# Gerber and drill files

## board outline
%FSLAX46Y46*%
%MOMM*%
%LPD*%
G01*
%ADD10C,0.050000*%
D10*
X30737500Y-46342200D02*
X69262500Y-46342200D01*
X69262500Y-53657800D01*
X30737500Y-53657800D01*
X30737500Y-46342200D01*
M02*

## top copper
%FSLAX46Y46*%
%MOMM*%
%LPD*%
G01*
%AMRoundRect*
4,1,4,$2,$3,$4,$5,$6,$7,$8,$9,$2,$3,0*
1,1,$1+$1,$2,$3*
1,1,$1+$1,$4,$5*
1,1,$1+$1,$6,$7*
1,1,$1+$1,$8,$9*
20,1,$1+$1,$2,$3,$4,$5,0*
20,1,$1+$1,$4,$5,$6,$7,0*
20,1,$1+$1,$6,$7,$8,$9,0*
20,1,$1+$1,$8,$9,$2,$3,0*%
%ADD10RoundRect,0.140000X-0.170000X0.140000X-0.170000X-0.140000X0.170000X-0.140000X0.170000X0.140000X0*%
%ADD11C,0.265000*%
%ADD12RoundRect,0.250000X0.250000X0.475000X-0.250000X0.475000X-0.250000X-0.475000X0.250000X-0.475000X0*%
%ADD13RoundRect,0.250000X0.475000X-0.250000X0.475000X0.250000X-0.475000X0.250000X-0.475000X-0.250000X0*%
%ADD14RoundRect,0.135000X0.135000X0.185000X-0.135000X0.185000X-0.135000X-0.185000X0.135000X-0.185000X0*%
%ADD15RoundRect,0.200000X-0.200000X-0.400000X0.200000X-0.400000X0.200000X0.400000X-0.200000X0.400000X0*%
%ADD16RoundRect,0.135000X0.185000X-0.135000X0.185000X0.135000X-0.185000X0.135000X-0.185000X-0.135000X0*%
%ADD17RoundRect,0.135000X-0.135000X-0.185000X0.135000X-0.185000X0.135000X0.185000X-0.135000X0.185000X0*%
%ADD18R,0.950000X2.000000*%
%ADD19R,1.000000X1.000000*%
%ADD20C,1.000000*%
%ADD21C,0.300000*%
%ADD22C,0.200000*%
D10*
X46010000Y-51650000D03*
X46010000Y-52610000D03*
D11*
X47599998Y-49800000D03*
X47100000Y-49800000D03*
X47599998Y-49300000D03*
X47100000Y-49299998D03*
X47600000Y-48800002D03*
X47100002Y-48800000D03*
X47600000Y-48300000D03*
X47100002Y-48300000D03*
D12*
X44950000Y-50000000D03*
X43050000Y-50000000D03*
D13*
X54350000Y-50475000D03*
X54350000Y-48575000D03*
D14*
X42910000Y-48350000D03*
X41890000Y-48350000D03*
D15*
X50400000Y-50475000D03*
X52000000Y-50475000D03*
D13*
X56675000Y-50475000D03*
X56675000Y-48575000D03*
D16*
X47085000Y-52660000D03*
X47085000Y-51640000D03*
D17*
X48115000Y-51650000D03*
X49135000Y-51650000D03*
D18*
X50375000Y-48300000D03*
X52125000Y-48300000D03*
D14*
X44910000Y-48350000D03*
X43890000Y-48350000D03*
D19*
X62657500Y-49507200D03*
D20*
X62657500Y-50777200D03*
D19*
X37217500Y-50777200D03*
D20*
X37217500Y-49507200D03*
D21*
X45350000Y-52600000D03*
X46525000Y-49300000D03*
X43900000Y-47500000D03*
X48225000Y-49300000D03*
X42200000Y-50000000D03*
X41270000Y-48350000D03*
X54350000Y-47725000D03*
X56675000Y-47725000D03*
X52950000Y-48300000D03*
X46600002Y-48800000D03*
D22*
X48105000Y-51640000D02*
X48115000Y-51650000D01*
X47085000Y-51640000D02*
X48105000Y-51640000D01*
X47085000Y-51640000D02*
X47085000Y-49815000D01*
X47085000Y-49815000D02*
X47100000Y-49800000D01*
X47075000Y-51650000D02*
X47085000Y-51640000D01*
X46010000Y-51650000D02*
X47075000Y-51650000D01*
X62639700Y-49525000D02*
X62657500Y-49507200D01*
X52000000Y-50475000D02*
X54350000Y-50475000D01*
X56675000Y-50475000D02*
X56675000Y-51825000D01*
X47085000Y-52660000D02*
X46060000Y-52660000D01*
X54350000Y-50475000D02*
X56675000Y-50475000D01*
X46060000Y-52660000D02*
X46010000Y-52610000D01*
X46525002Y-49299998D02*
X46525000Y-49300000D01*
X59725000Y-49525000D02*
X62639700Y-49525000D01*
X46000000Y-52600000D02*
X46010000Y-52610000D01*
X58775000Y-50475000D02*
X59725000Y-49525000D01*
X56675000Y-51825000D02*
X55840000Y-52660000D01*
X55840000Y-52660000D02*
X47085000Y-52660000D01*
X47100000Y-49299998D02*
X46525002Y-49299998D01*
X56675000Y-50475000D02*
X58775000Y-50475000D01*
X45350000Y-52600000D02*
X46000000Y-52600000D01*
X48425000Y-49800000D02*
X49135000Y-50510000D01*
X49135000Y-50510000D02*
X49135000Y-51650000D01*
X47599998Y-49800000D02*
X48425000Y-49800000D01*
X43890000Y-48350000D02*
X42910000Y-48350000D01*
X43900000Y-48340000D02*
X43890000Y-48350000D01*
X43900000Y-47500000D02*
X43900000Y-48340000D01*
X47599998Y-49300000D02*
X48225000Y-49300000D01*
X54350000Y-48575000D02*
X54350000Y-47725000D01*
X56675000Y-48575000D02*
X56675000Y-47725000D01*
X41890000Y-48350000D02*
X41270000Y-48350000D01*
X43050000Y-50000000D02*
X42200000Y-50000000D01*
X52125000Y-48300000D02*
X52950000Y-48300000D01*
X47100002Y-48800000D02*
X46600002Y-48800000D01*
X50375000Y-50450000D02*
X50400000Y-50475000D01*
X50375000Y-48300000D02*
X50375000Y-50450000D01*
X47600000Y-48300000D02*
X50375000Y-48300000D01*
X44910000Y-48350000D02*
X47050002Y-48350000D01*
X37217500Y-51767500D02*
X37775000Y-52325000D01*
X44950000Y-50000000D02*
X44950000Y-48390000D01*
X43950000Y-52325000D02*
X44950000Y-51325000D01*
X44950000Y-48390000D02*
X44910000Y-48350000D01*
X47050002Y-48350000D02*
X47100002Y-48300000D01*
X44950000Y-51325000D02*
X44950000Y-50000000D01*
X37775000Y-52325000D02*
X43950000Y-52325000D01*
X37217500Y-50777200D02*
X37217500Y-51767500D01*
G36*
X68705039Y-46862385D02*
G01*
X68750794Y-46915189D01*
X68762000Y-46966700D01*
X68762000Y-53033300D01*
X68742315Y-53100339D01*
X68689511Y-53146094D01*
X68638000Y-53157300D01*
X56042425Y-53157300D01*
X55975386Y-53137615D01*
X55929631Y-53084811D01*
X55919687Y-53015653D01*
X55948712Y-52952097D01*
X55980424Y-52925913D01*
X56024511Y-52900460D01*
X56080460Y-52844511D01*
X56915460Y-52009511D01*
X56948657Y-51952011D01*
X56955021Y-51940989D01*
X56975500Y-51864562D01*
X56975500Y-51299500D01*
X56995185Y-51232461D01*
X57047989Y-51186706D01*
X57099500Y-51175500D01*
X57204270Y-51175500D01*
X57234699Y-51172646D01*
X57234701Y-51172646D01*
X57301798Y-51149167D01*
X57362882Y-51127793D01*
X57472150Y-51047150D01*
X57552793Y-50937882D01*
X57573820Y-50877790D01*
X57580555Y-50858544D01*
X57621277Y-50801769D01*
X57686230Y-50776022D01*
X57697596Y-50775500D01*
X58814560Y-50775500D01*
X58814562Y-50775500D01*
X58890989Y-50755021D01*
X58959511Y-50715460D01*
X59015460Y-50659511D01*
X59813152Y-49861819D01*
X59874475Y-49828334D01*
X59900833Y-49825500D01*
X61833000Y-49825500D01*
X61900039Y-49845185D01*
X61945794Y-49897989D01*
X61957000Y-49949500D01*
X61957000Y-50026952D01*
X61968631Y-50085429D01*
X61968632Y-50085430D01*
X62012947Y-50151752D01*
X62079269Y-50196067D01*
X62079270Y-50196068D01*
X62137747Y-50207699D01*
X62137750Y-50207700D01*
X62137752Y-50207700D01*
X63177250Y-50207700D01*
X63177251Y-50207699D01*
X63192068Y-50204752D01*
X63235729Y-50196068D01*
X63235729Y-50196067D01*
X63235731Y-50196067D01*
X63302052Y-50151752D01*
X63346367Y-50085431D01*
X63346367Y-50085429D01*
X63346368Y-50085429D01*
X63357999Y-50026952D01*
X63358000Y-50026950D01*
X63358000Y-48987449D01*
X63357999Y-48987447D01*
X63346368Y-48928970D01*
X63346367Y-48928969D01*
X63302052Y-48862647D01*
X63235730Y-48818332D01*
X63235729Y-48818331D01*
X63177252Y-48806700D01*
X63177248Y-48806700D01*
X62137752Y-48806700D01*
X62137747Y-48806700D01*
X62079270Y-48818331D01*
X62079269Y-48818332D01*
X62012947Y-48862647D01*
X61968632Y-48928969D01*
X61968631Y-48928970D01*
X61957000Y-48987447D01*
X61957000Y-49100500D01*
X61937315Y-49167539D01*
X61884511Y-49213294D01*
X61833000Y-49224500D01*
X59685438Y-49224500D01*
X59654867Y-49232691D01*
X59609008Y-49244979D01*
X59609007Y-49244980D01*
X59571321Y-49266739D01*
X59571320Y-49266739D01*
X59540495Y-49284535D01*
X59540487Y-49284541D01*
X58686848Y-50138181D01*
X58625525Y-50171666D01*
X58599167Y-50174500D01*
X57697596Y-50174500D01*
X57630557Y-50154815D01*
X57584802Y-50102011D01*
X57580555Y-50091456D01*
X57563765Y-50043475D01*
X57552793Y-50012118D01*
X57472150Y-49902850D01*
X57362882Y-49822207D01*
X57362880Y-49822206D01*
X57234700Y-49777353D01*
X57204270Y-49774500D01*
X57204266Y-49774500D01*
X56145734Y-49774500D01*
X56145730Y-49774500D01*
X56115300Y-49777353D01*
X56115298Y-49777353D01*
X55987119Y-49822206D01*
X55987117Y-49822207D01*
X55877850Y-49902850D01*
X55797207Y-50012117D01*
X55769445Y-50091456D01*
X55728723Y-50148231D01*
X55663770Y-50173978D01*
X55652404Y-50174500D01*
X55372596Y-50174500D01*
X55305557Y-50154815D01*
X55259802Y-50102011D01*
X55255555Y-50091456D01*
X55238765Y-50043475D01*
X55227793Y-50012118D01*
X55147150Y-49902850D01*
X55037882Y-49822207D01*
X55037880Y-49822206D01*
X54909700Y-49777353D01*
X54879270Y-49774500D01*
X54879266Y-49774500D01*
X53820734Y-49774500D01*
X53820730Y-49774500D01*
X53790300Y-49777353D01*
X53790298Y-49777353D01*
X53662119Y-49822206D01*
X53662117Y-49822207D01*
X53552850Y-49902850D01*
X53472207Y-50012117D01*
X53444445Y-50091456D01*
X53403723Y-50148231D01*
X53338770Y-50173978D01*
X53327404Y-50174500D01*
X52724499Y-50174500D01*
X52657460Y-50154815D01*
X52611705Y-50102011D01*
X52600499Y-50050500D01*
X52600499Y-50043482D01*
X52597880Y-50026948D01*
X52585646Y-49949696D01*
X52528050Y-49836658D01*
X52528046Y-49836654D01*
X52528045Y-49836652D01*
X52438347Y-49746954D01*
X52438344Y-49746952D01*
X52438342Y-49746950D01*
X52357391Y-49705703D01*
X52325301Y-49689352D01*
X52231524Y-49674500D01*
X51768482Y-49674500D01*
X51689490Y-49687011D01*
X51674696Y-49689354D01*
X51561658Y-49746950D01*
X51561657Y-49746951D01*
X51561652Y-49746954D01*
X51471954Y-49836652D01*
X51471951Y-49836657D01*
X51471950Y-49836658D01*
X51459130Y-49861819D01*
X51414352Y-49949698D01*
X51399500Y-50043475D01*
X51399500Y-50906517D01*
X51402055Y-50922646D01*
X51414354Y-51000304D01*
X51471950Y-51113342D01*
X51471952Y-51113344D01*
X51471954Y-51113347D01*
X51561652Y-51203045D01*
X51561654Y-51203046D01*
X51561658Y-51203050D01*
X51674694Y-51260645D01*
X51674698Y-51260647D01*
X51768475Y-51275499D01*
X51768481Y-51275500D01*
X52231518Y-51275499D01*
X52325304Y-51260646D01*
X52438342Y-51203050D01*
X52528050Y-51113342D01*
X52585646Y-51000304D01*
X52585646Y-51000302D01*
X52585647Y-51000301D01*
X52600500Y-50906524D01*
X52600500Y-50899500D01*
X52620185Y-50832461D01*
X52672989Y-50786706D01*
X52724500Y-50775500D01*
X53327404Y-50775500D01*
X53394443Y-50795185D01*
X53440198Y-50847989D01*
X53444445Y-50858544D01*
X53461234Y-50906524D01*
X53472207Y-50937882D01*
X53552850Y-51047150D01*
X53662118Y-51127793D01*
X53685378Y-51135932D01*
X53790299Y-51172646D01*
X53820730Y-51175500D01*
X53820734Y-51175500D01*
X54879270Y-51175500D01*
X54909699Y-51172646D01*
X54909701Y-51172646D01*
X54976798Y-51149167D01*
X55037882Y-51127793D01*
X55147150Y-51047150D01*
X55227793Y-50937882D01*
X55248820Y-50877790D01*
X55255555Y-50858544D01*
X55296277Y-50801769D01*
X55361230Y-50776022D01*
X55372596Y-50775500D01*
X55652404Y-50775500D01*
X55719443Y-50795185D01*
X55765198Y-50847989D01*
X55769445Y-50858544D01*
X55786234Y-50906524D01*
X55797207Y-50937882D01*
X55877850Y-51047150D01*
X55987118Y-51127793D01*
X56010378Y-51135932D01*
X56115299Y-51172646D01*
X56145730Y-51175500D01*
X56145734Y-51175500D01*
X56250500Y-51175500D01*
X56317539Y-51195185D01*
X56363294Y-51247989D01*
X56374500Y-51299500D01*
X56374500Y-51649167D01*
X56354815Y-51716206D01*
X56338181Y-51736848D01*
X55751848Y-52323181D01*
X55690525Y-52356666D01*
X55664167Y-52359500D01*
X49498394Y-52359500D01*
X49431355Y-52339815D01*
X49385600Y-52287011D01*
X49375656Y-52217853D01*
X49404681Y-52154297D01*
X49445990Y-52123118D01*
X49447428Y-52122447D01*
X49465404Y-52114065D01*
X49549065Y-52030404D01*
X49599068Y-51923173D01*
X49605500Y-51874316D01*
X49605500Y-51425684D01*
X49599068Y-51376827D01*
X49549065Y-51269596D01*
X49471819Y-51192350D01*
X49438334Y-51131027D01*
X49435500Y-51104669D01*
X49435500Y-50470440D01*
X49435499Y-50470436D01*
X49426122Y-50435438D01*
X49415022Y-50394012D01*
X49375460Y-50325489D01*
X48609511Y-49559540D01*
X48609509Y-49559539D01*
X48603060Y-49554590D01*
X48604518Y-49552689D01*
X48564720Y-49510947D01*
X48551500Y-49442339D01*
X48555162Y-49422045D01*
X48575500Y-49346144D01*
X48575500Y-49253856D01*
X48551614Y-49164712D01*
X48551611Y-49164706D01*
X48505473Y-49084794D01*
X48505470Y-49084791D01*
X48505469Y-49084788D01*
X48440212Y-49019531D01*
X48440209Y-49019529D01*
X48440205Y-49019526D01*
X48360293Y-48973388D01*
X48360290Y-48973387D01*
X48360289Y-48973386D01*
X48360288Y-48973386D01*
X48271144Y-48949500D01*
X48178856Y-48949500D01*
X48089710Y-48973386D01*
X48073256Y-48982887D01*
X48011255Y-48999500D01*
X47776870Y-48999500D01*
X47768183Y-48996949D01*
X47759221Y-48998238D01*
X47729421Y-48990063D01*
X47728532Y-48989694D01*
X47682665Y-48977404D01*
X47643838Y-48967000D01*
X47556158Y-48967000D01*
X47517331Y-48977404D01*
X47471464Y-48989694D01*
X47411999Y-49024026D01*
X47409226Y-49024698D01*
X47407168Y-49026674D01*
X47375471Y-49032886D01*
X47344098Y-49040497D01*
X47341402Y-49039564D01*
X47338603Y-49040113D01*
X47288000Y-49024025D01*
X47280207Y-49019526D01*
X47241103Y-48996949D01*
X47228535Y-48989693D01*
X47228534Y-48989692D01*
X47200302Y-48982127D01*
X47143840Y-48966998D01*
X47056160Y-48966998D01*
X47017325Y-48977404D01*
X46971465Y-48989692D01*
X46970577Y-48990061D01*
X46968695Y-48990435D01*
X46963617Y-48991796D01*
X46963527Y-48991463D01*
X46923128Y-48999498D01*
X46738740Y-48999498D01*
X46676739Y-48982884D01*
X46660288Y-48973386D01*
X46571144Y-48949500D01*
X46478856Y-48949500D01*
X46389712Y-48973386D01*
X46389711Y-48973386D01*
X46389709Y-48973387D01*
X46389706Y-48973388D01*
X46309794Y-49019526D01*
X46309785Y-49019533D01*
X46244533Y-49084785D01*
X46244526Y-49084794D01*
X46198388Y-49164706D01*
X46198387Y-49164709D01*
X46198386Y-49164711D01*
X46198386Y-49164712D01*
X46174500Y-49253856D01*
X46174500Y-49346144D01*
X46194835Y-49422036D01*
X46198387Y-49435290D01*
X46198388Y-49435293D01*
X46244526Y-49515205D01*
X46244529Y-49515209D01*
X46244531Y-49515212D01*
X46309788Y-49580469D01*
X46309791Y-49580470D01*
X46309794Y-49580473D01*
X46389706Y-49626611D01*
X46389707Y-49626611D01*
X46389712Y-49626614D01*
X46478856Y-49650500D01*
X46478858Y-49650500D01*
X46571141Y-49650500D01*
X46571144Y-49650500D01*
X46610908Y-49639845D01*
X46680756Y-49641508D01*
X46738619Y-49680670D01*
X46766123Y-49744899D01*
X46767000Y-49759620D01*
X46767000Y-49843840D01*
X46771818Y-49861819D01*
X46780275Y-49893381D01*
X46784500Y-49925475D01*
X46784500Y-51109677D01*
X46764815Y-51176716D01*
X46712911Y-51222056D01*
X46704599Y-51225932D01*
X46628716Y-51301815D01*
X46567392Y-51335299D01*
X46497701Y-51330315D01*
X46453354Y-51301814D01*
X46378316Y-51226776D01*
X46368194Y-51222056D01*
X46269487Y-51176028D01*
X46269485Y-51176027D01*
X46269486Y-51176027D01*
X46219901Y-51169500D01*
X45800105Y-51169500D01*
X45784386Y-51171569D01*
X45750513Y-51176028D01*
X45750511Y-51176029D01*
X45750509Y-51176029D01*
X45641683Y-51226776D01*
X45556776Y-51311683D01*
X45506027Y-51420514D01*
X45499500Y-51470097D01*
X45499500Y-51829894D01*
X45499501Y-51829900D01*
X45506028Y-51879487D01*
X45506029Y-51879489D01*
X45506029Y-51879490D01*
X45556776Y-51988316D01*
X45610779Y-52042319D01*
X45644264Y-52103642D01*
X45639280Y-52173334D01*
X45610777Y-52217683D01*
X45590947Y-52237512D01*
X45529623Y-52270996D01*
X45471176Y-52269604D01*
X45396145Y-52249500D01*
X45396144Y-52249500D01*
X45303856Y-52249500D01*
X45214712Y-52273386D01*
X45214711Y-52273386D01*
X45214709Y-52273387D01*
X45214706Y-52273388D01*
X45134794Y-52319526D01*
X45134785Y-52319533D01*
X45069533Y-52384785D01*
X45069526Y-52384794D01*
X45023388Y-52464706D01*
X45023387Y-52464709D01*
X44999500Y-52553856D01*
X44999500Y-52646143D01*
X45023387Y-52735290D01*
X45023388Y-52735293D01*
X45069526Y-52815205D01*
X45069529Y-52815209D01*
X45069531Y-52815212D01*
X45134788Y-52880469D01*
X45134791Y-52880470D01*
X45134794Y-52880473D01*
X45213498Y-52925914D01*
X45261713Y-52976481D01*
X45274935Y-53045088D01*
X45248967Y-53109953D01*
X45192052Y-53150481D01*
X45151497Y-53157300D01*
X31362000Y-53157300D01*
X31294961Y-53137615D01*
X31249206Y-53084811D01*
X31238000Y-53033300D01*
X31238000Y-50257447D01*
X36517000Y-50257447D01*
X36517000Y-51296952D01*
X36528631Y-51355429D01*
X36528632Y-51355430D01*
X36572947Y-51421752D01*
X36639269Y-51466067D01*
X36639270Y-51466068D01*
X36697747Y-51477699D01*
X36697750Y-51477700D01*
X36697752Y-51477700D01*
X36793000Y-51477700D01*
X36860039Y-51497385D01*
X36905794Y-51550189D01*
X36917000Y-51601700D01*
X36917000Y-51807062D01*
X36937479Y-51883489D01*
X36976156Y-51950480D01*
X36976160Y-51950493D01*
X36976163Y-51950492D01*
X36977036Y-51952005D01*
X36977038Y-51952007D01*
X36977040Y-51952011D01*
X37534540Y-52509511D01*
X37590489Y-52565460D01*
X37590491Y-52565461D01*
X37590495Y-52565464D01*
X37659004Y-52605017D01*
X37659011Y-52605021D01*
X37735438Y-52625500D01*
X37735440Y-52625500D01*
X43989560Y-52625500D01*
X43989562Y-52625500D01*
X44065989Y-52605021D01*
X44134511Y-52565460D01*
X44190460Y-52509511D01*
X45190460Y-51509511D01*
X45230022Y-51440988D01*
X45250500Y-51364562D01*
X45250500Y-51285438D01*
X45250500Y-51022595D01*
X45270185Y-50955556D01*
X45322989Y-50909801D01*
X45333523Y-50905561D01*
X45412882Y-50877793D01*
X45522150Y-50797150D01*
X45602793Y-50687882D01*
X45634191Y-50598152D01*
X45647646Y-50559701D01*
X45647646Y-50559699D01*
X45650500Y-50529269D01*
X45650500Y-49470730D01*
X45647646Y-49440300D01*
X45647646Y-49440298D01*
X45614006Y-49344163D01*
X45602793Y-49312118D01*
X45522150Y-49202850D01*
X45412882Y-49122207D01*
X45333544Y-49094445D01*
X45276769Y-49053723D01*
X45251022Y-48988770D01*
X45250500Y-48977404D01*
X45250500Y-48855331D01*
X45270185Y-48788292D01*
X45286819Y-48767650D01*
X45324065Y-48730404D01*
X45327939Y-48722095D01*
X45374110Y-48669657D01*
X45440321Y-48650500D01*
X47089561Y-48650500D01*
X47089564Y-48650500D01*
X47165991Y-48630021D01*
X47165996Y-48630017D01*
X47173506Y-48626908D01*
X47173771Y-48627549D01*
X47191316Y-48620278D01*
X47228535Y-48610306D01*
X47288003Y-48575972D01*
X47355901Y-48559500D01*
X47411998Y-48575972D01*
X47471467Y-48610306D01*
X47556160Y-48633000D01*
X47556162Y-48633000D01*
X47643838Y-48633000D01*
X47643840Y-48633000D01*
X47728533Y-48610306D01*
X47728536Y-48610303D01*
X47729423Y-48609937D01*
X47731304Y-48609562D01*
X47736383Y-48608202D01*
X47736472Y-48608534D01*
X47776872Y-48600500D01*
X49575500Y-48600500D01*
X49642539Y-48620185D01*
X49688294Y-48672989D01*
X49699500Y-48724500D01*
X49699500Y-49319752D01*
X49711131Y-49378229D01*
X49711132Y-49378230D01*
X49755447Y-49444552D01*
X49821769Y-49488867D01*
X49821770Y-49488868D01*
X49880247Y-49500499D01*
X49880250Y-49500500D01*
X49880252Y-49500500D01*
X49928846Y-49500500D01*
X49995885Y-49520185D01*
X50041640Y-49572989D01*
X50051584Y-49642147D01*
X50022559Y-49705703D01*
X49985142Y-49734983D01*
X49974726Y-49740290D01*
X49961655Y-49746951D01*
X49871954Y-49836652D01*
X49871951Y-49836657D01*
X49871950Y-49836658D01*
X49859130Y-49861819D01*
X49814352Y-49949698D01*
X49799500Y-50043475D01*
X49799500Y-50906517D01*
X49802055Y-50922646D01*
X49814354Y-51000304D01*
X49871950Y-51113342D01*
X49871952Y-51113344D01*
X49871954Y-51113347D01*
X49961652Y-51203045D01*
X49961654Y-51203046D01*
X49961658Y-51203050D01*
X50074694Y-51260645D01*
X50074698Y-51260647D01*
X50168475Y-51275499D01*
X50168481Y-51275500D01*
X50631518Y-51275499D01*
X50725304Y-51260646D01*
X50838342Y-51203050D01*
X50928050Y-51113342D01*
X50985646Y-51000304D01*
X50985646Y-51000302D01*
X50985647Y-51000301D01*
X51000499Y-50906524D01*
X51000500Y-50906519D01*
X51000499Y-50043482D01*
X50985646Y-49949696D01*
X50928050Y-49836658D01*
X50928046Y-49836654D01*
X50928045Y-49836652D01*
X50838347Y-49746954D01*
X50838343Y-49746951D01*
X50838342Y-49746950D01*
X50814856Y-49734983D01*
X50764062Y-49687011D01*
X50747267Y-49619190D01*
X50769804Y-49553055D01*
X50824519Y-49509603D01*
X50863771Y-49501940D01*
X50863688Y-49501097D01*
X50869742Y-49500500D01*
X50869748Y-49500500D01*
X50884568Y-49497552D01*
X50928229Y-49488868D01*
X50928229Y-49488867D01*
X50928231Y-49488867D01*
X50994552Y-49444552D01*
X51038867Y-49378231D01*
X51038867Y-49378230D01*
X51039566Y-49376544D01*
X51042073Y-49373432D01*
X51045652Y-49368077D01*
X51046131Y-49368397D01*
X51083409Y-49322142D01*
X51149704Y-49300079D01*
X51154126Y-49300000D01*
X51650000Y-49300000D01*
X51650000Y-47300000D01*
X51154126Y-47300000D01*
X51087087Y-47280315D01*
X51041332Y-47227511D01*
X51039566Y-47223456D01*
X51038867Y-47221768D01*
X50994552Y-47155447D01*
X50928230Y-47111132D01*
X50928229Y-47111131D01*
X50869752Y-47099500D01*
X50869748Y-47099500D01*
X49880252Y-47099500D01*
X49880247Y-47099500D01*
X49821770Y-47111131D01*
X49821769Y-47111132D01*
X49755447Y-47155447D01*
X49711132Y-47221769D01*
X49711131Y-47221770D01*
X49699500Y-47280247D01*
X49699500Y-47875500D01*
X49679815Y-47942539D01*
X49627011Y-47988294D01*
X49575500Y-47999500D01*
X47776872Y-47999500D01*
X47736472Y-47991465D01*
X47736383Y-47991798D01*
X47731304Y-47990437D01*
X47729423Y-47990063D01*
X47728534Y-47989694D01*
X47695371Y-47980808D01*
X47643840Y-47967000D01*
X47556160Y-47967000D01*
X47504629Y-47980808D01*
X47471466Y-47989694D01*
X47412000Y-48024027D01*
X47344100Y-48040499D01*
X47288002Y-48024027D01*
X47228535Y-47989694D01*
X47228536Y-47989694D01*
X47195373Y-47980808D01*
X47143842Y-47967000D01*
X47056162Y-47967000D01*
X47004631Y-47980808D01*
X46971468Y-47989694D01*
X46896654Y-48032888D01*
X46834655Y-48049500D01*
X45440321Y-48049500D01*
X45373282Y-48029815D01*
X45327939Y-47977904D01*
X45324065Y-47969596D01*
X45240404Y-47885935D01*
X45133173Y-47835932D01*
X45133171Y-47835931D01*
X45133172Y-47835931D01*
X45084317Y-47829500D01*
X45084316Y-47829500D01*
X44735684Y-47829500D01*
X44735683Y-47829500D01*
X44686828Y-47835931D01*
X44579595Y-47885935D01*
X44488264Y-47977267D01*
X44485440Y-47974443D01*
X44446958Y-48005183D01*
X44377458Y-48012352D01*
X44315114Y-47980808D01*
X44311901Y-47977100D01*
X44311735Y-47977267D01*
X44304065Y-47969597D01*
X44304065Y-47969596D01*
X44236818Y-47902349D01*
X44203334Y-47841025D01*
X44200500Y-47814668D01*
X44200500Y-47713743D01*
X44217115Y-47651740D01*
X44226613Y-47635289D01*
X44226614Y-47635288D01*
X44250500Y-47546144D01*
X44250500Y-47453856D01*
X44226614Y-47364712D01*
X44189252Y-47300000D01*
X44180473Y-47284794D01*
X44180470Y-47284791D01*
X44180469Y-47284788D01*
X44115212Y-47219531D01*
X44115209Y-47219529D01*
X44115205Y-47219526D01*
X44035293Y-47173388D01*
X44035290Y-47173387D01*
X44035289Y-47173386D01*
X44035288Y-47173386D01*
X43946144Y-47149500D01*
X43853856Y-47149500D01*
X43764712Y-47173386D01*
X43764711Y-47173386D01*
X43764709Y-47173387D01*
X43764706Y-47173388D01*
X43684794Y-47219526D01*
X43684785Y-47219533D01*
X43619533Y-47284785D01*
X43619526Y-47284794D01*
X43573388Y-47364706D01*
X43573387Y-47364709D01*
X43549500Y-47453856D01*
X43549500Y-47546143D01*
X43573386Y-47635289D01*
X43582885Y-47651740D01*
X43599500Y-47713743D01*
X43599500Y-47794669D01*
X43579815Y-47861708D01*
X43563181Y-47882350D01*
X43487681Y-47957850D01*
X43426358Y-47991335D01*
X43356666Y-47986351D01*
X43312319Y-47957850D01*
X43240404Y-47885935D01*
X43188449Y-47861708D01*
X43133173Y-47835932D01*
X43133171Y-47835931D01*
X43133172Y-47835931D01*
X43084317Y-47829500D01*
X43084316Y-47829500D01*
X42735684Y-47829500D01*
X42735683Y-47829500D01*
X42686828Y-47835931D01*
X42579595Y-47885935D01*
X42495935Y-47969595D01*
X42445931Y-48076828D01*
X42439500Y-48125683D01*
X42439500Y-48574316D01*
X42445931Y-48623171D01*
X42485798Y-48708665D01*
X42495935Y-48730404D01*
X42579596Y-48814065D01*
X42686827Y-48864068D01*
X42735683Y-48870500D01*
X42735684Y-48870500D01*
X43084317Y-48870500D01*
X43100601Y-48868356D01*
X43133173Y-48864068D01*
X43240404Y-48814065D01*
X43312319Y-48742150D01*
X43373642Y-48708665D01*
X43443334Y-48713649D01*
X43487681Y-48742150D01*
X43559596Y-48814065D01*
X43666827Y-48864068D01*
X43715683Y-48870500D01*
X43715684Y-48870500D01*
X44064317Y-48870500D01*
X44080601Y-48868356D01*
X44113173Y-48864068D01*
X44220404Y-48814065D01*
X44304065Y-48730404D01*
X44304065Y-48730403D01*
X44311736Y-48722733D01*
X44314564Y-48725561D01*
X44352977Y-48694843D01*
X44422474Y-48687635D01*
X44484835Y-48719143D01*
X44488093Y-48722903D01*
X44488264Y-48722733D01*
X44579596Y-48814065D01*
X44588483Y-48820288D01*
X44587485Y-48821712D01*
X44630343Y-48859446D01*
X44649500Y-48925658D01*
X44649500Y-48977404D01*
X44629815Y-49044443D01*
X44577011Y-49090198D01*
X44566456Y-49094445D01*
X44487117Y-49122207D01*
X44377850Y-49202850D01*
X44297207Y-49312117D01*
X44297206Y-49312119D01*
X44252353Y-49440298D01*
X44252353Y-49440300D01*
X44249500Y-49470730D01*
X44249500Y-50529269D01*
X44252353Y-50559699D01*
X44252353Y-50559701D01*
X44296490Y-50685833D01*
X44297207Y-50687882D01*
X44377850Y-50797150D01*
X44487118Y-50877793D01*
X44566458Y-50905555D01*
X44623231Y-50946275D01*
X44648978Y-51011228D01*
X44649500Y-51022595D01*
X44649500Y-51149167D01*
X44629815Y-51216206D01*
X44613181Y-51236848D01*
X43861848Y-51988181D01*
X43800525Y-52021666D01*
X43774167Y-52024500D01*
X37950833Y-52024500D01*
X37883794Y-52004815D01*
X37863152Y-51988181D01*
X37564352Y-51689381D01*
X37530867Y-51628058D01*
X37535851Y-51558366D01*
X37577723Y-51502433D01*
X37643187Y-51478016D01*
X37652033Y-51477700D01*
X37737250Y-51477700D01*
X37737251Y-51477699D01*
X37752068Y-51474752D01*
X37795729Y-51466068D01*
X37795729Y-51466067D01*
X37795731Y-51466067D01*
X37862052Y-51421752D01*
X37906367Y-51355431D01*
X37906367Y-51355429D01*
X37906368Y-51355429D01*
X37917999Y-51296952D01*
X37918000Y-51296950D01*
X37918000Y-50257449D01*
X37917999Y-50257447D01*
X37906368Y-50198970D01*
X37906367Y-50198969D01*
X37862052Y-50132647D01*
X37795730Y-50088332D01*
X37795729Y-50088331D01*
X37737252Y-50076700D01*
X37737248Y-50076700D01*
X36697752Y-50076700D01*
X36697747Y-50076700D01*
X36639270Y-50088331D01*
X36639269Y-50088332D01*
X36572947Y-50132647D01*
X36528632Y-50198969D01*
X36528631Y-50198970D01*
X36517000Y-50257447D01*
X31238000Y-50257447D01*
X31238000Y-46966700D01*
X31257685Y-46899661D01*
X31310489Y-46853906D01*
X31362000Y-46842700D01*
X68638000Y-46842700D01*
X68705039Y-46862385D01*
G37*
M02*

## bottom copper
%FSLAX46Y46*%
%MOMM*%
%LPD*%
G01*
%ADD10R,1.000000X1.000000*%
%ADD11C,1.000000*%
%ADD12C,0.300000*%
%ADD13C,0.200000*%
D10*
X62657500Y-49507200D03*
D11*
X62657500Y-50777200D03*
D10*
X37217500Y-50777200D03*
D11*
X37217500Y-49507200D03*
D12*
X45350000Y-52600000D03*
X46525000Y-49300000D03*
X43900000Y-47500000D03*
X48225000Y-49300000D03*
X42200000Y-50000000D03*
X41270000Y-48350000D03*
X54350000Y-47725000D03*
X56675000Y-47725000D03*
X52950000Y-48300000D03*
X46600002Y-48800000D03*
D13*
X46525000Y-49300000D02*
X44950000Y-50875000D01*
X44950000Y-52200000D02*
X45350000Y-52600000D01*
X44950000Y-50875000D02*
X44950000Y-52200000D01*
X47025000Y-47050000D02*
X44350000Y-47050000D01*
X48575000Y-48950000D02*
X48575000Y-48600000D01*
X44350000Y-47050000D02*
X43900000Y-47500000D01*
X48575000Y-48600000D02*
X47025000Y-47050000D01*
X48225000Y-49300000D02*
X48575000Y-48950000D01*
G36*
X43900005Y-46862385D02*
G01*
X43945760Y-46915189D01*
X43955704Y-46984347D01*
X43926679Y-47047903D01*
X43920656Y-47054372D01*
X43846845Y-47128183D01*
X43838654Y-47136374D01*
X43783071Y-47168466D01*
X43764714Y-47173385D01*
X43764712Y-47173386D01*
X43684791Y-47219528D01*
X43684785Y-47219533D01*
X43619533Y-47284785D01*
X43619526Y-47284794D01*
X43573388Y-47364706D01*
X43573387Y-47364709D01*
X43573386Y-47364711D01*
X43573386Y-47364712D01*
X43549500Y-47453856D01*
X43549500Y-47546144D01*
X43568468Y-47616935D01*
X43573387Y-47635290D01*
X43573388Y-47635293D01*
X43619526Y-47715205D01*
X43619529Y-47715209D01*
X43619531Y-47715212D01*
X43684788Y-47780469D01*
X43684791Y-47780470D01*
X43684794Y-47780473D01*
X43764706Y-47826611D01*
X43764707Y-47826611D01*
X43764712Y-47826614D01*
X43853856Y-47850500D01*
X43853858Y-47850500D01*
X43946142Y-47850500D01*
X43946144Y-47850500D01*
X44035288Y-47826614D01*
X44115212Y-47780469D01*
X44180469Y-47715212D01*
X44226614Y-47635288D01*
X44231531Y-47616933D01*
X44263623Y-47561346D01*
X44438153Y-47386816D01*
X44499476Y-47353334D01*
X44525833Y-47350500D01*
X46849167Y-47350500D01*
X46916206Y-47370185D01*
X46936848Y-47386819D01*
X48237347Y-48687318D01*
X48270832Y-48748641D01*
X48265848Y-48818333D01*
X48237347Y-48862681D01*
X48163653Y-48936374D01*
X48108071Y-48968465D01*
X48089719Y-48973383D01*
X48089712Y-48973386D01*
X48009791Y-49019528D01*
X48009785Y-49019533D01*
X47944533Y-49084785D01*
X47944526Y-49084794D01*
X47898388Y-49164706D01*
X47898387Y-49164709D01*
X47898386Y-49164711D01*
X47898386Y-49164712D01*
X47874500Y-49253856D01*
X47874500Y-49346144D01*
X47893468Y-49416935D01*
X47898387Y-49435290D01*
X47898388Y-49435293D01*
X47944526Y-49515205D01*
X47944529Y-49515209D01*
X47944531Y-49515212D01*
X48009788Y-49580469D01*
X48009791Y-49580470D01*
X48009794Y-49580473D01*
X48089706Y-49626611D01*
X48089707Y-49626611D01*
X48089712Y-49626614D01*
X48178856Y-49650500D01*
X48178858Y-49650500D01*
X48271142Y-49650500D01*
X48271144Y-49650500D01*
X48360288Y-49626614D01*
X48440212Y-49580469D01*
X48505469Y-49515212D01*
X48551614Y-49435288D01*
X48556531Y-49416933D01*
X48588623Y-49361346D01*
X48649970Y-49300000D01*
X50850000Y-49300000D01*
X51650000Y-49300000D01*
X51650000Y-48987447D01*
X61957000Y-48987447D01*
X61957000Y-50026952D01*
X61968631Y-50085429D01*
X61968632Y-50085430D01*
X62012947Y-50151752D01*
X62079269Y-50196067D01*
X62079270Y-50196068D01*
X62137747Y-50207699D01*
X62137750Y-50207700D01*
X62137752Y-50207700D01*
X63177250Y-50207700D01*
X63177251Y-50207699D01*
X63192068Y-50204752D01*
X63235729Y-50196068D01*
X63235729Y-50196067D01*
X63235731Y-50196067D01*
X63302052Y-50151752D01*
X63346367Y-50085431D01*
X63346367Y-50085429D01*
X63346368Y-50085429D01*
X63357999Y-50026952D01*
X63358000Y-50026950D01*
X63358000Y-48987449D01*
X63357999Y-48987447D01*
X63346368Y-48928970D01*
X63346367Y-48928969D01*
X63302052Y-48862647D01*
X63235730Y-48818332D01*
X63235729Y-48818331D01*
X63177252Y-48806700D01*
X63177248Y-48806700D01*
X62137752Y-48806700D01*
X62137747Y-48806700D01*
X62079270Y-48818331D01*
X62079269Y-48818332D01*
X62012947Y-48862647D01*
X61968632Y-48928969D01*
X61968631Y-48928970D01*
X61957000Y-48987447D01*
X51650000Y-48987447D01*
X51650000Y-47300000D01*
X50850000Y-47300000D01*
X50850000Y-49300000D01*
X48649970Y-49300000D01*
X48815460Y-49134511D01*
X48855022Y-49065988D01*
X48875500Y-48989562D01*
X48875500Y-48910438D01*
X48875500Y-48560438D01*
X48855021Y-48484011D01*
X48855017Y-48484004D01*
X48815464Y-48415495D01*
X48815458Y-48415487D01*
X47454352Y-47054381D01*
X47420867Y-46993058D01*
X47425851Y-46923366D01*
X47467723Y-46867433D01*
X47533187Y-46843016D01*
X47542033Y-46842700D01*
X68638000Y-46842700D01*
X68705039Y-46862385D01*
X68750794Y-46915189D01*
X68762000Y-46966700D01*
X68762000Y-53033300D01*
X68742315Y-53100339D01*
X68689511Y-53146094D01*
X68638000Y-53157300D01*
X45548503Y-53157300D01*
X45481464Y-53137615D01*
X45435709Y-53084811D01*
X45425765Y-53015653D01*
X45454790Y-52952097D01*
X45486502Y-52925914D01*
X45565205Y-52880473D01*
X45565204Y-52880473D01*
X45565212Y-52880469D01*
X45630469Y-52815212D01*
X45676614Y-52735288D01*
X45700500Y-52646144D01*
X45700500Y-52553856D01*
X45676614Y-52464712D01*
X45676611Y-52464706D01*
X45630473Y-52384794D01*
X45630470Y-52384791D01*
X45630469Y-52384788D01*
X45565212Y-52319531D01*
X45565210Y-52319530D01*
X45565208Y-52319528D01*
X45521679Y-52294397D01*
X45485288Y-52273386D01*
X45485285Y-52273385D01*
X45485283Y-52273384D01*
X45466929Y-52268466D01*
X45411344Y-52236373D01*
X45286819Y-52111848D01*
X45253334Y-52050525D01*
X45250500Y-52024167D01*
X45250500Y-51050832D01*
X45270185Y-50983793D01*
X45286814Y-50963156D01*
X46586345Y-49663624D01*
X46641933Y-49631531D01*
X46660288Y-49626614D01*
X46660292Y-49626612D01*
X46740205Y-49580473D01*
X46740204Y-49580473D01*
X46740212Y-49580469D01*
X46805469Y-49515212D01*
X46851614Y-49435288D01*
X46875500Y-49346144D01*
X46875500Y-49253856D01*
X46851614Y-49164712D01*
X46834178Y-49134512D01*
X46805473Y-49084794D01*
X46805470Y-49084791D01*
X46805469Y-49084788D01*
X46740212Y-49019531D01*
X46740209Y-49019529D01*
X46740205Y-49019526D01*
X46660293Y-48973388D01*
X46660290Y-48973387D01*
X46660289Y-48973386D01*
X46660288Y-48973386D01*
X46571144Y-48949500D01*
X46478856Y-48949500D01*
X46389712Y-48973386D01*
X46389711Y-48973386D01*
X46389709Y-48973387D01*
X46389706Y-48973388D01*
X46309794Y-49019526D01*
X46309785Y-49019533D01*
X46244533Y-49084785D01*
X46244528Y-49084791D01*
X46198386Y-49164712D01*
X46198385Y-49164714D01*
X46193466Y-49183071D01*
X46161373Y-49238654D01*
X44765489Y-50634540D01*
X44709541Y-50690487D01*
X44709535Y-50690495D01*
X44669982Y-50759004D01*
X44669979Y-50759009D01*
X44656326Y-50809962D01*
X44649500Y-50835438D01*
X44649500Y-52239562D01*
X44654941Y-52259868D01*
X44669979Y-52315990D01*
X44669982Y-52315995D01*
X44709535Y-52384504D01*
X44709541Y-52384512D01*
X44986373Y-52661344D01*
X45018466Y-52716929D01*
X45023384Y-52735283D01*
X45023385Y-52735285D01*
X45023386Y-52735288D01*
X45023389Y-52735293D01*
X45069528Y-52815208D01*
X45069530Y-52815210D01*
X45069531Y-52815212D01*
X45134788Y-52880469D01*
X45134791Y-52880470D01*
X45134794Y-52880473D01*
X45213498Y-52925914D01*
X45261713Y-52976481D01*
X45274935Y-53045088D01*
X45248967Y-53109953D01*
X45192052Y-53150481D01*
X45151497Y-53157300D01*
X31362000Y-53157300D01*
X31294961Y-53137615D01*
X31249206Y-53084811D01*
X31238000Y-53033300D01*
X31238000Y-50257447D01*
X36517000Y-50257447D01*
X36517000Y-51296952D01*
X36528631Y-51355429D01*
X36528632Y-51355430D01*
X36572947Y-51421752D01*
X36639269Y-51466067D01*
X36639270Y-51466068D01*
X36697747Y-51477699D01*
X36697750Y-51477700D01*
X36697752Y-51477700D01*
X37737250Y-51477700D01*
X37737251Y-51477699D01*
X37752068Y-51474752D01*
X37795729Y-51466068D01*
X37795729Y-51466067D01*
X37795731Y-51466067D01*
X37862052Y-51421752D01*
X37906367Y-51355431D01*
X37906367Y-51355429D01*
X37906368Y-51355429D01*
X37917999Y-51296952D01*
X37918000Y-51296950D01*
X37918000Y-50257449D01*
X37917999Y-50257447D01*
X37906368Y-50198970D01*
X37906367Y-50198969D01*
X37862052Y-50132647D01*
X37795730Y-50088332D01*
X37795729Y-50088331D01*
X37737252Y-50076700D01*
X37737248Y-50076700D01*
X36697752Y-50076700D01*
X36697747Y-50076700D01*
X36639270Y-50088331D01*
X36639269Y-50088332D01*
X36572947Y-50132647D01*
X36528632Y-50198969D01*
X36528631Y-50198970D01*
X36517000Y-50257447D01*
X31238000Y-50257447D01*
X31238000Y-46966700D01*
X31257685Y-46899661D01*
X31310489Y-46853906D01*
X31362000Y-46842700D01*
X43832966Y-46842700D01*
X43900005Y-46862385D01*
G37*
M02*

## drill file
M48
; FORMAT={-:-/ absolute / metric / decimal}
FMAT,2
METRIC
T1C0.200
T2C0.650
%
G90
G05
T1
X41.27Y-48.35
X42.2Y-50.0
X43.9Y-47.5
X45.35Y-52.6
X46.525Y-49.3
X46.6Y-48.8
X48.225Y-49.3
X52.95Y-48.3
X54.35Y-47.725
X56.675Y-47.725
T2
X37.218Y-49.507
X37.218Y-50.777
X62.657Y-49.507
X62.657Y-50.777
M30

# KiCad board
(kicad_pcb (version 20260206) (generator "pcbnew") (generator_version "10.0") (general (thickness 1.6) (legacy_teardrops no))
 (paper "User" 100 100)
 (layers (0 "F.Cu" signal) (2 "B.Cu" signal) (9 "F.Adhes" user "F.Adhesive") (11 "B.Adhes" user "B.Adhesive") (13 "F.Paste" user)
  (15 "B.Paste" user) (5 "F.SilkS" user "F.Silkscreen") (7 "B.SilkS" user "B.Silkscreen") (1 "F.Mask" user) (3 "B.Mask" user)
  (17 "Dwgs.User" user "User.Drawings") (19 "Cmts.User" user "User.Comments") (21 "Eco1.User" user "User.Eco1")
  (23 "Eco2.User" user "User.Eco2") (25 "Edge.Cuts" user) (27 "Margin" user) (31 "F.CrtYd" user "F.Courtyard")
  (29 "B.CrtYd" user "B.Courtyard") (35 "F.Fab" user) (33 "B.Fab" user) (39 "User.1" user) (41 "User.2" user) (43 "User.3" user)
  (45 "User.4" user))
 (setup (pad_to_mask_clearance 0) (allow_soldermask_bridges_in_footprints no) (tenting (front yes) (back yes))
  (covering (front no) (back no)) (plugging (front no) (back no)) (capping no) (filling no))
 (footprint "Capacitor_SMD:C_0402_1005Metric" (layer "F.Cu") (at 46.01 52.13 -90)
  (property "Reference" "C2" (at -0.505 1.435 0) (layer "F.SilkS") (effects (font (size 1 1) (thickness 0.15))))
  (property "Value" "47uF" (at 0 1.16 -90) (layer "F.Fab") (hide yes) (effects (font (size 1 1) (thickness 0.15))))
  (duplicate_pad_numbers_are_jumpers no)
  (pad "1" smd roundrect (at -0.48 0 -90) (size 0.56 0.62) (layers "F.Cu" "F.Mask" "F.Paste") (roundrect_rratio 0.25) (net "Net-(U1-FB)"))
  (pad "2" smd roundrect (at 0.48 0 -90) (size 0.56 0.62) (layers "F.Cu" "F.Mask" "F.Paste") (roundrect_rratio 0.25) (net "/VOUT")))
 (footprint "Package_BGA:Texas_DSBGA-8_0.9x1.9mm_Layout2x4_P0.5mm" (layer "F.Cu") (at 47.35 49.05 180)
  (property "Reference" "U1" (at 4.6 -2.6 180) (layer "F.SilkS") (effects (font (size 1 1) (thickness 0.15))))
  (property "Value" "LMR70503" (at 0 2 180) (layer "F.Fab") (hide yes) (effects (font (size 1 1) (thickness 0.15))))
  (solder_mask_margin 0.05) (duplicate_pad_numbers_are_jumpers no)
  (pad "" smd rect (at -0.25 0.249998 180) (size 0.3 0.3) (layers "F.Paste"))
  (pad "" smd rect (at -0.25 0.75 180) (size 0.3 0.3) (layers "F.Paste"))
  (pad "" smd rect (at -0.249998 -0.75 180) (size 0.3 0.3) (layers "F.Paste"))
  (pad "" smd rect (at -0.249998 -0.25 180) (size 0.3 0.3) (layers "F.Paste"))
  (pad "" smd rect (at 0.249998 0.25 180) (size 0.3 0.3) (layers "F.Paste"))
  (pad "" smd rect (at 0.249998 0.75 180) (size 0.3 0.3) (layers "F.Paste"))
  (pad "" smd rect (at 0.25 -0.75 180) (size 0.3 0.3) (layers "F.Paste"))
  (pad "" smd rect (at 0.25 -0.249998 180) (size 0.3 0.3) (layers "F.Paste"))
  (pad "A1" smd circle (at -0.249998 -0.75 180) (size 0.265 0.265) (layers "F.Cu" "F.Mask") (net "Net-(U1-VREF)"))
  (pad "A2" smd circle (at 0.25 -0.75 180) (size 0.265 0.265) (layers "F.Cu" "F.Mask") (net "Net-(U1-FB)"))
  (pad "B1" smd circle (at -0.249998 -0.25 180) (size 0.265 0.265) (layers "F.Cu" "F.Mask") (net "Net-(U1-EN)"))
  (pad "B2" smd circle (at 0.25 -0.249998 180) (size 0.265 0.265) (layers "F.Cu" "F.Mask") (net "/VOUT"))
  (pad "C1" smd circle (at -0.25 0.249998 180) (size 0.265 0.265) (layers "F.Cu" "F.Mask") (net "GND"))
  (pad "C2" smd circle (at 0.249998 0.25 180) (size 0.265 0.265) (layers "F.Cu" "F.Mask") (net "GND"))
  (pad "D1" smd circle (at -0.25 0.75 180) (size 0.265 0.265) (layers "F.Cu" "F.Mask") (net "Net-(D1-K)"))
  (pad "D2" smd circle (at 0.249998 0.75 180) (size 0.265 0.265) (layers "F.Cu" "F.Mask") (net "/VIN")))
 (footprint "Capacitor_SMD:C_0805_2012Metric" (layer "F.Cu") (at 44 50 180)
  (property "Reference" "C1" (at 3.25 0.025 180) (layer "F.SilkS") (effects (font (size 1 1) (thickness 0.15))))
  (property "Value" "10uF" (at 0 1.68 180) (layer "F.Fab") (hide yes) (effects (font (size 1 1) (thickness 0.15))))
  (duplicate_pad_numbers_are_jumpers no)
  (pad "1" smd roundrect (at -0.95 0 180) (size 1 1.45) (layers "F.Cu" "F.Mask" "F.Paste") (roundrect_rratio 0.25) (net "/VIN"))
  (pad "2" smd roundrect (at 0.95 0 180) (size 1 1.45) (layers "F.Cu" "F.Mask" "F.Paste") (roundrect_rratio 0.25) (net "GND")))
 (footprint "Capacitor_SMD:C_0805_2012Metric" (layer "F.Cu") (at 54.35 49.525 90)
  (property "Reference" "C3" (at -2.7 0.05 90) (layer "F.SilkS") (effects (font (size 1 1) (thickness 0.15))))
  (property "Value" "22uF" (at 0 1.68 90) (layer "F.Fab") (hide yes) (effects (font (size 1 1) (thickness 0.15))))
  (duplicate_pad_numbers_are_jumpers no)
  (pad "1" smd roundrect (at -0.95 0 90) (size 1 1.45) (layers "F.Cu" "F.Mask" "F.Paste") (roundrect_rratio 0.25) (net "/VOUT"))
  (pad "2" smd roundrect (at 0.95 0 90) (size 1 1.45) (layers "F.Cu" "F.Mask" "F.Paste") (roundrect_rratio 0.25) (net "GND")))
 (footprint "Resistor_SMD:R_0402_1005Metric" (layer "F.Cu") (at 42.4 48.35 180)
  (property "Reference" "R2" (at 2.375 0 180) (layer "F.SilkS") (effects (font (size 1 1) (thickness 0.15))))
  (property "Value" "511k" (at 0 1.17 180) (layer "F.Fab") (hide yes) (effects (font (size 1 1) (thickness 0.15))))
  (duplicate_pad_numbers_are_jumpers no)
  (pad "1" smd roundrect (at -0.51 0 180) (size 0.54 0.64) (layers "F.Cu" "F.Mask" "F.Paste") (roundrect_rratio 0.25) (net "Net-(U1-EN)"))
  (pad "2" smd roundrect (at 0.51 0 180) (size 0.54 0.64) (layers "F.Cu" "F.Mask" "F.Paste") (roundrect_rratio 0.25) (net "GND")))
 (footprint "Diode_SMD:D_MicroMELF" (layer "F.Cu") (at 51.2 50.475)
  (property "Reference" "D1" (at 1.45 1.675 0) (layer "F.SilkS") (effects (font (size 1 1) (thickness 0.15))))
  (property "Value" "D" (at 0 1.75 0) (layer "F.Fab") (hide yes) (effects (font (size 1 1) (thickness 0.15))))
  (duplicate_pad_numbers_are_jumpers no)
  (pad "1" smd roundrect (at -0.8 0) (size 0.8 1.2) (layers "F.Cu" "F.Mask" "F.Paste") (roundrect_rratio 0.25) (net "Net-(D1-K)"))
  (pad "2" smd roundrect (at 0.8 0) (size 0.8 1.2) (layers "F.Cu" "F.Mask" "F.Paste") (roundrect_rratio 0.25) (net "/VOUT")))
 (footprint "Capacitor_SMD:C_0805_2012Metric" (layer "F.Cu") (at 56.675 49.525 90)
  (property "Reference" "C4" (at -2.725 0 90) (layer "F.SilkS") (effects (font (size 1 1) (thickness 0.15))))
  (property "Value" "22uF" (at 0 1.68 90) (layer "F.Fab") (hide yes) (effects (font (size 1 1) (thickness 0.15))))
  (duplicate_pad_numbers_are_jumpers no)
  (pad "1" smd roundrect (at -0.95 0 90) (size 1 1.45) (layers "F.Cu" "F.Mask" "F.Paste") (roundrect_rratio 0.25) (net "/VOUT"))
  (pad "2" smd roundrect (at 0.95 0 90) (size 1 1.45) (layers "F.Cu" "F.Mask" "F.Paste") (roundrect_rratio 0.25) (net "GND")))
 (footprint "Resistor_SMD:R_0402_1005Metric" (layer "F.Cu") (at 47.085 52.15 90)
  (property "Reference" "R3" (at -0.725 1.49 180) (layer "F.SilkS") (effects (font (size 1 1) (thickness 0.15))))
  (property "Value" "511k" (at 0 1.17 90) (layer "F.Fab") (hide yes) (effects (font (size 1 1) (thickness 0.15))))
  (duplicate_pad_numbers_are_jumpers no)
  (pad "1" smd roundrect (at -0.51 0 90) (size 0.54 0.64) (layers "F.Cu" "F.Mask" "F.Paste") (roundrect_rratio 0.25) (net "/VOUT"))
  (pad "2" smd roundrect (at 0.51 0 90) (size 0.54 0.64) (layers "F.Cu" "F.Mask" "F.Paste") (roundrect_rratio 0.25) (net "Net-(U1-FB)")))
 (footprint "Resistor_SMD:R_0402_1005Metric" (layer "F.Cu") (at 48.625 51.65)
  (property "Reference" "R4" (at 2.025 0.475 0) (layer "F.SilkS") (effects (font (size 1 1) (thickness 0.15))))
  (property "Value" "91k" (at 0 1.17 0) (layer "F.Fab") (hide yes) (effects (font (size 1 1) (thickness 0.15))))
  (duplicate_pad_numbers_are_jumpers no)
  (pad "1" smd roundrect (at -0.51 0) (size 0.54 0.64) (layers "F.Cu" "F.Mask" "F.Paste") (roundrect_rratio 0.25) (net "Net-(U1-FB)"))
  (pad "2" smd roundrect (at 0.51 0) (size 0.54 0.64) (layers "F.Cu" "F.Mask" "F.Paste") (roundrect_rratio 0.25) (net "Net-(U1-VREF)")))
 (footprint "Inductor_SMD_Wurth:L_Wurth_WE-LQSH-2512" (layer "F.Cu") (at 51.25 48.3)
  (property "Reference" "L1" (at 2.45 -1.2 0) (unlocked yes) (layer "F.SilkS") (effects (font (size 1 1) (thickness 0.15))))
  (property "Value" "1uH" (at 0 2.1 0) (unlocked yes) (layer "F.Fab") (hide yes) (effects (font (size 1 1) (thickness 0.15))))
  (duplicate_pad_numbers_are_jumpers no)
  (pad "1" smd rect (at -0.875 0) (size 0.95 2) (layers "F.Cu" "F.Mask" "F.Paste") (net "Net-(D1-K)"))
  (pad "2" smd rect (at 0.875 0) (size 0.95 2) (layers "F.Cu" "F.Mask" "F.Paste") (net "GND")))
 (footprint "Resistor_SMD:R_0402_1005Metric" (layer "F.Cu") (at 44.4 48.35 180)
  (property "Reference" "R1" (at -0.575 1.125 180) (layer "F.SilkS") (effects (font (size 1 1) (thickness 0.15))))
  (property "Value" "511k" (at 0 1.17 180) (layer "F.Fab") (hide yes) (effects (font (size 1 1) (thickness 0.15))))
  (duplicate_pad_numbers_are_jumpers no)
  (pad "1" smd roundrect (at -0.51 0 180) (size 0.54 0.64) (layers "F.Cu" "F.Mask" "F.Paste") (roundrect_rratio 0.25) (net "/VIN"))
  (pad "2" smd roundrect (at 0.51 0 180) (size 0.54 0.64) (layers "F.Cu" "F.Mask" "F.Paste") (roundrect_rratio 0.25) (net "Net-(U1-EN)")))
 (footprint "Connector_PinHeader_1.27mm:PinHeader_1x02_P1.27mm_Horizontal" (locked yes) (layer "F.Cu") (at 65.0875 50.1422)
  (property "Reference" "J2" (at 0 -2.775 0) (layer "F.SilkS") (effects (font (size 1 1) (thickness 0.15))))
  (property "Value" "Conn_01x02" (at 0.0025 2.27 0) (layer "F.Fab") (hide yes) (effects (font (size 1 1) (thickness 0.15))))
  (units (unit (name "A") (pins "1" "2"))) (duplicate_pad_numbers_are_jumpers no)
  (pad "1" thru_hole rect (at -2.43 -0.635) (size 1 1) (drill 0.65) (layers "*.Cu" "*.Mask") (remove_unused_layers no) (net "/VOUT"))
  (pad "2" thru_hole circle (at -2.43 0.635) (size 1 1) (drill 0.65) (layers "*.Cu" "*.Mask") (remove_unused_layers no) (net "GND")))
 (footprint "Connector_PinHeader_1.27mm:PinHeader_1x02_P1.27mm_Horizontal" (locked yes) (layer "F.Cu") (at 34.7875 50.1422 180)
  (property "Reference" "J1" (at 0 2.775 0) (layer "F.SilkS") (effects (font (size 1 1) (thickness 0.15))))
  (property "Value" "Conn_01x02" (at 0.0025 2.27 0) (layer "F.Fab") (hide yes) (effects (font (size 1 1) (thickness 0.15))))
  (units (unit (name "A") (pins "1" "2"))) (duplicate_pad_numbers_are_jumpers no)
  (pad "1" thru_hole rect (at -2.43 -0.635 180) (size 1 1) (drill 0.65) (layers "*.Cu" "*.Mask") (remove_unused_layers no) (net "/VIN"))
  (pad "2" thru_hole circle (at -2.43 0.635 180) (size 1 1) (drill 0.65) (layers "*.Cu" "*.Mask") (remove_unused_layers no) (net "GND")))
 (gr_rect (start 30.7375 46.3422) (end 69.2625 53.6578) (stroke (width 0.05) (type solid)) (fill no) (locked yes) (layer "Edge.Cuts"))
 (segment (start 48.105 51.64) (end 48.115 51.65) (width 0.2) (layer "F.Cu") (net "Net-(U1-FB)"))
 (segment (start 47.085 51.64) (end 48.105 51.64) (width 0.2) (layer "F.Cu") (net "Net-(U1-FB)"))
 (segment (start 47.085 51.64) (end 47.085 49.815) (width 0.2) (layer "F.Cu") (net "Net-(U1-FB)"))
 (segment (start 47.085 49.815) (end 47.1 49.8) (width 0.2) (layer "F.Cu") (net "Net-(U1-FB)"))
 (segment (start 47.075 51.65) (end 47.085 51.64) (width 0.2) (layer "F.Cu") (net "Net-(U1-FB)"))
 (segment (start 46.01 51.65) (end 47.075 51.65) (width 0.2) (layer "F.Cu") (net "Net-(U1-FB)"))
 (segment (start 62.6397 49.525) (end 62.6575 49.5072) (width 0.2) (layer "F.Cu") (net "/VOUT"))
 (segment (start 52 50.475) (end 54.35 50.475) (width 0.2) (layer "F.Cu") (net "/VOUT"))
 (segment (start 56.675 50.475) (end 56.675 51.825) (width 0.2) (layer "F.Cu") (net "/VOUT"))
 (segment (start 47.085 52.66) (end 46.06 52.66) (width 0.2) (layer "F.Cu") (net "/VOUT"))
 (segment (start 54.35 50.475) (end 56.675 50.475) (width 0.2) (layer "F.Cu") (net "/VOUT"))
 (segment (start 46.06 52.66) (end 46.01 52.61) (width 0.2) (layer "F.Cu") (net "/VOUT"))
 (segment (start 46.525002 49.299998) (end 46.525 49.3) (width 0.2) (layer "F.Cu") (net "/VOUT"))
 (segment (start 59.725 49.525) (end 62.6397 49.525) (width 0.2) (layer "F.Cu") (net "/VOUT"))
 (segment (start 46 52.6) (end 46.01 52.61) (width 0.2) (layer "F.Cu") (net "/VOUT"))
 (segment (start 58.775 50.475) (end 59.725 49.525) (width 0.2) (layer "F.Cu") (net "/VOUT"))
 (segment (start 56.675 51.825) (end 55.84 52.66) (width 0.2) (layer "F.Cu") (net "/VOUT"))
 (segment (start 55.84 52.66) (end 47.085 52.66) (width 0.2) (layer "F.Cu") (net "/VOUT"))
 (segment (start 47.1 49.299998) (end 46.525002 49.299998) (width 0.2) (layer "F.Cu") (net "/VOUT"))
 (segment (start 56.675 50.475) (end 58.775 50.475) (width 0.2) (layer "F.Cu") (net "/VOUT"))
 (segment (start 45.35 52.6) (end 46 52.6) (width 0.2) (layer "F.Cu") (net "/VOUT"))
 (via (at 45.35 52.6) (size 0.3) (drill 0.2) (layers "F.Cu" "B.Cu") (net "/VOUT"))
 (via (at 46.525 49.3) (size 0.3) (drill 0.2) (layers "F.Cu" "B.Cu") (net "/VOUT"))
 (segment (start 46.525 49.3) (end 44.95 50.875) (width 0.2) (layer "B.Cu") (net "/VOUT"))
 (segment (start 44.95 52.2) (end 45.35 52.6) (width 0.2) (layer "B.Cu") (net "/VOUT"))
 (segment (start 44.95 50.875) (end 44.95 52.2) (width 0.2) (layer "B.Cu") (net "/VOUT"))
 (segment (start 48.425 49.8) (end 49.135 50.51) (width 0.2) (layer "F.Cu") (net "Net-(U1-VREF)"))
 (segment (start 49.135 50.51) (end 49.135 51.65) (width 0.2) (layer "F.Cu") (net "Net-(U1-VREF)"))
 (segment (start 47.599998 49.8) (end 48.425 49.8) (width 0.2) (layer "F.Cu") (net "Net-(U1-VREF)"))
 (segment (start 43.89 48.35) (end 42.91 48.35) (width 0.2) (layer "F.Cu") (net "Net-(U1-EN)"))
 (segment (start 43.9 48.34) (end 43.89 48.35) (width 0.2) (layer "F.Cu") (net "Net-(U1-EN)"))
 (segment (start 43.9 47.5) (end 43.9 48.34) (width 0.2) (layer "F.Cu") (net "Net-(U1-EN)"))
 (segment (start 47.599998 49.3) (end 48.225 49.3) (width 0.2) (layer "F.Cu") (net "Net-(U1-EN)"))
 (via (at 43.9 47.5) (size 0.3) (drill 0.2) (layers "F.Cu" "B.Cu") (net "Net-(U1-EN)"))
 (via (at 48.225 49.3) (size 0.3) (drill 0.2) (layers "F.Cu" "B.Cu") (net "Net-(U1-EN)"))
 (segment (start 47.025 47.05) (end 44.35 47.05) (width 0.2) (layer "B.Cu") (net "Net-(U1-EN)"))
 (segment (start 48.575 48.95) (end 48.575 48.6) (width 0.2) (layer "B.Cu") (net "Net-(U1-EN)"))
 (segment (start 44.35 47.05) (end 43.9 47.5) (width 0.2) (layer "B.Cu") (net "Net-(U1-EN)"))
 (segment (start 48.575 48.6) (end 47.025 47.05) (width 0.2) (layer "B.Cu") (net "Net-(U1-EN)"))
 (segment (start 48.225 49.3) (end 48.575 48.95) (width 0.2) (layer "B.Cu") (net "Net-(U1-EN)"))
 (segment (start 54.35 48.575) (end 54.35 47.725) (width 0.2) (layer "F.Cu") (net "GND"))
 (segment (start 56.675 48.575) (end 56.675 47.725) (width 0.2) (layer "F.Cu") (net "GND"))
 (segment (start 41.89 48.35) (end 41.27 48.35) (width 0.2) (layer "F.Cu") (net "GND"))
 (segment (start 43.05 50) (end 42.2 50) (width 0.2) (layer "F.Cu") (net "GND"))
 (segment (start 52.125 48.3) (end 52.95 48.3) (width 0.2) (layer "F.Cu") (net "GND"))
 (segment (start 47.100002 48.8) (end 46.600002 48.8) (width 0.2) (layer "F.Cu") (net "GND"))
 (via (at 42.2 50) (size 0.3) (drill 0.2) (layers "F.Cu" "B.Cu") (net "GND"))
 (via (at 41.27 48.35) (size 0.3) (drill 0.2) (layers "F.Cu" "B.Cu") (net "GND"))
 (via (at 54.35 47.725) (size 0.3) (drill 0.2) (layers "F.Cu" "B.Cu") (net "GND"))
 (via (at 56.675 47.725) (size 0.3) (drill 0.2) (layers "F.Cu" "B.Cu") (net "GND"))
 (via (at 52.95 48.3) (size 0.3) (drill 0.2) (layers "F.Cu" "B.Cu") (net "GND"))
 (via (at 46.600002 48.8) (size 0.3) (drill 0.2) (layers "F.Cu" "B.Cu") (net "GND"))
 (segment (start 50.375 50.45) (end 50.4 50.475) (width 0.2) (layer "F.Cu") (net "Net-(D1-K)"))
 (segment (start 50.375 48.3) (end 50.375 50.45) (width 0.2) (layer "F.Cu") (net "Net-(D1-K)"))
 (segment (start 47.6 48.3) (end 50.375 48.3) (width 0.2) (layer "F.Cu") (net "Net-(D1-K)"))
 (segment (start 44.91 48.35) (end 47.050002 48.35) (width 0.2) (layer "F.Cu") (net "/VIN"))
 (segment (start 37.2175 51.7675) (end 37.775 52.325) (width 0.2) (layer "F.Cu") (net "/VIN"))
 (segment (start 44.95 50) (end 44.95 48.39) (width 0.2) (layer "F.Cu") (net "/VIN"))
 (segment (start 43.95 52.325) (end 44.95 51.325) (width 0.2) (layer "F.Cu") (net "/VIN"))
 (segment (start 44.95 48.39) (end 44.91 48.35) (width 0.2) (layer "F.Cu") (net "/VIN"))
 (segment (start 47.050002 48.35) (end 47.100002 48.3) (width 0.2) (layer "F.Cu") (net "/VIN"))
 (segment (start 44.95 51.325) (end 44.95 50) (width 0.2) (layer "F.Cu") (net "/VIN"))
 (segment (start 37.775 52.325) (end 43.95 52.325) (width 0.2) (layer "F.Cu") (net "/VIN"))
 (segment (start 37.2175 50.7772) (end 37.2175 51.7675) (width 0.2) (layer "F.Cu") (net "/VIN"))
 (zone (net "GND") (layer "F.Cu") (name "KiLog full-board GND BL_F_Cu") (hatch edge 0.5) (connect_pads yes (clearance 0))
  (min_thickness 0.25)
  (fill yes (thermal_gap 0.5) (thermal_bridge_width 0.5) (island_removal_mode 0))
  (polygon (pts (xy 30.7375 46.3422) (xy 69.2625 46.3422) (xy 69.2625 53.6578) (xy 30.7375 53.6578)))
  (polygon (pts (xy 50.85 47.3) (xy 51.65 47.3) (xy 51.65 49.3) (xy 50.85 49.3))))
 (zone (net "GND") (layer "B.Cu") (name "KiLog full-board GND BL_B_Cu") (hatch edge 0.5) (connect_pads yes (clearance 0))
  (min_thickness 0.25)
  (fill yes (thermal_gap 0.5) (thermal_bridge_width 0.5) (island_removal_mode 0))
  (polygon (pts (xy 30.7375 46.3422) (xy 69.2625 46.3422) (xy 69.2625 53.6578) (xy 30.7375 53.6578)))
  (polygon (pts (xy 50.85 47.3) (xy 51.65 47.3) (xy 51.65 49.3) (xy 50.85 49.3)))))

